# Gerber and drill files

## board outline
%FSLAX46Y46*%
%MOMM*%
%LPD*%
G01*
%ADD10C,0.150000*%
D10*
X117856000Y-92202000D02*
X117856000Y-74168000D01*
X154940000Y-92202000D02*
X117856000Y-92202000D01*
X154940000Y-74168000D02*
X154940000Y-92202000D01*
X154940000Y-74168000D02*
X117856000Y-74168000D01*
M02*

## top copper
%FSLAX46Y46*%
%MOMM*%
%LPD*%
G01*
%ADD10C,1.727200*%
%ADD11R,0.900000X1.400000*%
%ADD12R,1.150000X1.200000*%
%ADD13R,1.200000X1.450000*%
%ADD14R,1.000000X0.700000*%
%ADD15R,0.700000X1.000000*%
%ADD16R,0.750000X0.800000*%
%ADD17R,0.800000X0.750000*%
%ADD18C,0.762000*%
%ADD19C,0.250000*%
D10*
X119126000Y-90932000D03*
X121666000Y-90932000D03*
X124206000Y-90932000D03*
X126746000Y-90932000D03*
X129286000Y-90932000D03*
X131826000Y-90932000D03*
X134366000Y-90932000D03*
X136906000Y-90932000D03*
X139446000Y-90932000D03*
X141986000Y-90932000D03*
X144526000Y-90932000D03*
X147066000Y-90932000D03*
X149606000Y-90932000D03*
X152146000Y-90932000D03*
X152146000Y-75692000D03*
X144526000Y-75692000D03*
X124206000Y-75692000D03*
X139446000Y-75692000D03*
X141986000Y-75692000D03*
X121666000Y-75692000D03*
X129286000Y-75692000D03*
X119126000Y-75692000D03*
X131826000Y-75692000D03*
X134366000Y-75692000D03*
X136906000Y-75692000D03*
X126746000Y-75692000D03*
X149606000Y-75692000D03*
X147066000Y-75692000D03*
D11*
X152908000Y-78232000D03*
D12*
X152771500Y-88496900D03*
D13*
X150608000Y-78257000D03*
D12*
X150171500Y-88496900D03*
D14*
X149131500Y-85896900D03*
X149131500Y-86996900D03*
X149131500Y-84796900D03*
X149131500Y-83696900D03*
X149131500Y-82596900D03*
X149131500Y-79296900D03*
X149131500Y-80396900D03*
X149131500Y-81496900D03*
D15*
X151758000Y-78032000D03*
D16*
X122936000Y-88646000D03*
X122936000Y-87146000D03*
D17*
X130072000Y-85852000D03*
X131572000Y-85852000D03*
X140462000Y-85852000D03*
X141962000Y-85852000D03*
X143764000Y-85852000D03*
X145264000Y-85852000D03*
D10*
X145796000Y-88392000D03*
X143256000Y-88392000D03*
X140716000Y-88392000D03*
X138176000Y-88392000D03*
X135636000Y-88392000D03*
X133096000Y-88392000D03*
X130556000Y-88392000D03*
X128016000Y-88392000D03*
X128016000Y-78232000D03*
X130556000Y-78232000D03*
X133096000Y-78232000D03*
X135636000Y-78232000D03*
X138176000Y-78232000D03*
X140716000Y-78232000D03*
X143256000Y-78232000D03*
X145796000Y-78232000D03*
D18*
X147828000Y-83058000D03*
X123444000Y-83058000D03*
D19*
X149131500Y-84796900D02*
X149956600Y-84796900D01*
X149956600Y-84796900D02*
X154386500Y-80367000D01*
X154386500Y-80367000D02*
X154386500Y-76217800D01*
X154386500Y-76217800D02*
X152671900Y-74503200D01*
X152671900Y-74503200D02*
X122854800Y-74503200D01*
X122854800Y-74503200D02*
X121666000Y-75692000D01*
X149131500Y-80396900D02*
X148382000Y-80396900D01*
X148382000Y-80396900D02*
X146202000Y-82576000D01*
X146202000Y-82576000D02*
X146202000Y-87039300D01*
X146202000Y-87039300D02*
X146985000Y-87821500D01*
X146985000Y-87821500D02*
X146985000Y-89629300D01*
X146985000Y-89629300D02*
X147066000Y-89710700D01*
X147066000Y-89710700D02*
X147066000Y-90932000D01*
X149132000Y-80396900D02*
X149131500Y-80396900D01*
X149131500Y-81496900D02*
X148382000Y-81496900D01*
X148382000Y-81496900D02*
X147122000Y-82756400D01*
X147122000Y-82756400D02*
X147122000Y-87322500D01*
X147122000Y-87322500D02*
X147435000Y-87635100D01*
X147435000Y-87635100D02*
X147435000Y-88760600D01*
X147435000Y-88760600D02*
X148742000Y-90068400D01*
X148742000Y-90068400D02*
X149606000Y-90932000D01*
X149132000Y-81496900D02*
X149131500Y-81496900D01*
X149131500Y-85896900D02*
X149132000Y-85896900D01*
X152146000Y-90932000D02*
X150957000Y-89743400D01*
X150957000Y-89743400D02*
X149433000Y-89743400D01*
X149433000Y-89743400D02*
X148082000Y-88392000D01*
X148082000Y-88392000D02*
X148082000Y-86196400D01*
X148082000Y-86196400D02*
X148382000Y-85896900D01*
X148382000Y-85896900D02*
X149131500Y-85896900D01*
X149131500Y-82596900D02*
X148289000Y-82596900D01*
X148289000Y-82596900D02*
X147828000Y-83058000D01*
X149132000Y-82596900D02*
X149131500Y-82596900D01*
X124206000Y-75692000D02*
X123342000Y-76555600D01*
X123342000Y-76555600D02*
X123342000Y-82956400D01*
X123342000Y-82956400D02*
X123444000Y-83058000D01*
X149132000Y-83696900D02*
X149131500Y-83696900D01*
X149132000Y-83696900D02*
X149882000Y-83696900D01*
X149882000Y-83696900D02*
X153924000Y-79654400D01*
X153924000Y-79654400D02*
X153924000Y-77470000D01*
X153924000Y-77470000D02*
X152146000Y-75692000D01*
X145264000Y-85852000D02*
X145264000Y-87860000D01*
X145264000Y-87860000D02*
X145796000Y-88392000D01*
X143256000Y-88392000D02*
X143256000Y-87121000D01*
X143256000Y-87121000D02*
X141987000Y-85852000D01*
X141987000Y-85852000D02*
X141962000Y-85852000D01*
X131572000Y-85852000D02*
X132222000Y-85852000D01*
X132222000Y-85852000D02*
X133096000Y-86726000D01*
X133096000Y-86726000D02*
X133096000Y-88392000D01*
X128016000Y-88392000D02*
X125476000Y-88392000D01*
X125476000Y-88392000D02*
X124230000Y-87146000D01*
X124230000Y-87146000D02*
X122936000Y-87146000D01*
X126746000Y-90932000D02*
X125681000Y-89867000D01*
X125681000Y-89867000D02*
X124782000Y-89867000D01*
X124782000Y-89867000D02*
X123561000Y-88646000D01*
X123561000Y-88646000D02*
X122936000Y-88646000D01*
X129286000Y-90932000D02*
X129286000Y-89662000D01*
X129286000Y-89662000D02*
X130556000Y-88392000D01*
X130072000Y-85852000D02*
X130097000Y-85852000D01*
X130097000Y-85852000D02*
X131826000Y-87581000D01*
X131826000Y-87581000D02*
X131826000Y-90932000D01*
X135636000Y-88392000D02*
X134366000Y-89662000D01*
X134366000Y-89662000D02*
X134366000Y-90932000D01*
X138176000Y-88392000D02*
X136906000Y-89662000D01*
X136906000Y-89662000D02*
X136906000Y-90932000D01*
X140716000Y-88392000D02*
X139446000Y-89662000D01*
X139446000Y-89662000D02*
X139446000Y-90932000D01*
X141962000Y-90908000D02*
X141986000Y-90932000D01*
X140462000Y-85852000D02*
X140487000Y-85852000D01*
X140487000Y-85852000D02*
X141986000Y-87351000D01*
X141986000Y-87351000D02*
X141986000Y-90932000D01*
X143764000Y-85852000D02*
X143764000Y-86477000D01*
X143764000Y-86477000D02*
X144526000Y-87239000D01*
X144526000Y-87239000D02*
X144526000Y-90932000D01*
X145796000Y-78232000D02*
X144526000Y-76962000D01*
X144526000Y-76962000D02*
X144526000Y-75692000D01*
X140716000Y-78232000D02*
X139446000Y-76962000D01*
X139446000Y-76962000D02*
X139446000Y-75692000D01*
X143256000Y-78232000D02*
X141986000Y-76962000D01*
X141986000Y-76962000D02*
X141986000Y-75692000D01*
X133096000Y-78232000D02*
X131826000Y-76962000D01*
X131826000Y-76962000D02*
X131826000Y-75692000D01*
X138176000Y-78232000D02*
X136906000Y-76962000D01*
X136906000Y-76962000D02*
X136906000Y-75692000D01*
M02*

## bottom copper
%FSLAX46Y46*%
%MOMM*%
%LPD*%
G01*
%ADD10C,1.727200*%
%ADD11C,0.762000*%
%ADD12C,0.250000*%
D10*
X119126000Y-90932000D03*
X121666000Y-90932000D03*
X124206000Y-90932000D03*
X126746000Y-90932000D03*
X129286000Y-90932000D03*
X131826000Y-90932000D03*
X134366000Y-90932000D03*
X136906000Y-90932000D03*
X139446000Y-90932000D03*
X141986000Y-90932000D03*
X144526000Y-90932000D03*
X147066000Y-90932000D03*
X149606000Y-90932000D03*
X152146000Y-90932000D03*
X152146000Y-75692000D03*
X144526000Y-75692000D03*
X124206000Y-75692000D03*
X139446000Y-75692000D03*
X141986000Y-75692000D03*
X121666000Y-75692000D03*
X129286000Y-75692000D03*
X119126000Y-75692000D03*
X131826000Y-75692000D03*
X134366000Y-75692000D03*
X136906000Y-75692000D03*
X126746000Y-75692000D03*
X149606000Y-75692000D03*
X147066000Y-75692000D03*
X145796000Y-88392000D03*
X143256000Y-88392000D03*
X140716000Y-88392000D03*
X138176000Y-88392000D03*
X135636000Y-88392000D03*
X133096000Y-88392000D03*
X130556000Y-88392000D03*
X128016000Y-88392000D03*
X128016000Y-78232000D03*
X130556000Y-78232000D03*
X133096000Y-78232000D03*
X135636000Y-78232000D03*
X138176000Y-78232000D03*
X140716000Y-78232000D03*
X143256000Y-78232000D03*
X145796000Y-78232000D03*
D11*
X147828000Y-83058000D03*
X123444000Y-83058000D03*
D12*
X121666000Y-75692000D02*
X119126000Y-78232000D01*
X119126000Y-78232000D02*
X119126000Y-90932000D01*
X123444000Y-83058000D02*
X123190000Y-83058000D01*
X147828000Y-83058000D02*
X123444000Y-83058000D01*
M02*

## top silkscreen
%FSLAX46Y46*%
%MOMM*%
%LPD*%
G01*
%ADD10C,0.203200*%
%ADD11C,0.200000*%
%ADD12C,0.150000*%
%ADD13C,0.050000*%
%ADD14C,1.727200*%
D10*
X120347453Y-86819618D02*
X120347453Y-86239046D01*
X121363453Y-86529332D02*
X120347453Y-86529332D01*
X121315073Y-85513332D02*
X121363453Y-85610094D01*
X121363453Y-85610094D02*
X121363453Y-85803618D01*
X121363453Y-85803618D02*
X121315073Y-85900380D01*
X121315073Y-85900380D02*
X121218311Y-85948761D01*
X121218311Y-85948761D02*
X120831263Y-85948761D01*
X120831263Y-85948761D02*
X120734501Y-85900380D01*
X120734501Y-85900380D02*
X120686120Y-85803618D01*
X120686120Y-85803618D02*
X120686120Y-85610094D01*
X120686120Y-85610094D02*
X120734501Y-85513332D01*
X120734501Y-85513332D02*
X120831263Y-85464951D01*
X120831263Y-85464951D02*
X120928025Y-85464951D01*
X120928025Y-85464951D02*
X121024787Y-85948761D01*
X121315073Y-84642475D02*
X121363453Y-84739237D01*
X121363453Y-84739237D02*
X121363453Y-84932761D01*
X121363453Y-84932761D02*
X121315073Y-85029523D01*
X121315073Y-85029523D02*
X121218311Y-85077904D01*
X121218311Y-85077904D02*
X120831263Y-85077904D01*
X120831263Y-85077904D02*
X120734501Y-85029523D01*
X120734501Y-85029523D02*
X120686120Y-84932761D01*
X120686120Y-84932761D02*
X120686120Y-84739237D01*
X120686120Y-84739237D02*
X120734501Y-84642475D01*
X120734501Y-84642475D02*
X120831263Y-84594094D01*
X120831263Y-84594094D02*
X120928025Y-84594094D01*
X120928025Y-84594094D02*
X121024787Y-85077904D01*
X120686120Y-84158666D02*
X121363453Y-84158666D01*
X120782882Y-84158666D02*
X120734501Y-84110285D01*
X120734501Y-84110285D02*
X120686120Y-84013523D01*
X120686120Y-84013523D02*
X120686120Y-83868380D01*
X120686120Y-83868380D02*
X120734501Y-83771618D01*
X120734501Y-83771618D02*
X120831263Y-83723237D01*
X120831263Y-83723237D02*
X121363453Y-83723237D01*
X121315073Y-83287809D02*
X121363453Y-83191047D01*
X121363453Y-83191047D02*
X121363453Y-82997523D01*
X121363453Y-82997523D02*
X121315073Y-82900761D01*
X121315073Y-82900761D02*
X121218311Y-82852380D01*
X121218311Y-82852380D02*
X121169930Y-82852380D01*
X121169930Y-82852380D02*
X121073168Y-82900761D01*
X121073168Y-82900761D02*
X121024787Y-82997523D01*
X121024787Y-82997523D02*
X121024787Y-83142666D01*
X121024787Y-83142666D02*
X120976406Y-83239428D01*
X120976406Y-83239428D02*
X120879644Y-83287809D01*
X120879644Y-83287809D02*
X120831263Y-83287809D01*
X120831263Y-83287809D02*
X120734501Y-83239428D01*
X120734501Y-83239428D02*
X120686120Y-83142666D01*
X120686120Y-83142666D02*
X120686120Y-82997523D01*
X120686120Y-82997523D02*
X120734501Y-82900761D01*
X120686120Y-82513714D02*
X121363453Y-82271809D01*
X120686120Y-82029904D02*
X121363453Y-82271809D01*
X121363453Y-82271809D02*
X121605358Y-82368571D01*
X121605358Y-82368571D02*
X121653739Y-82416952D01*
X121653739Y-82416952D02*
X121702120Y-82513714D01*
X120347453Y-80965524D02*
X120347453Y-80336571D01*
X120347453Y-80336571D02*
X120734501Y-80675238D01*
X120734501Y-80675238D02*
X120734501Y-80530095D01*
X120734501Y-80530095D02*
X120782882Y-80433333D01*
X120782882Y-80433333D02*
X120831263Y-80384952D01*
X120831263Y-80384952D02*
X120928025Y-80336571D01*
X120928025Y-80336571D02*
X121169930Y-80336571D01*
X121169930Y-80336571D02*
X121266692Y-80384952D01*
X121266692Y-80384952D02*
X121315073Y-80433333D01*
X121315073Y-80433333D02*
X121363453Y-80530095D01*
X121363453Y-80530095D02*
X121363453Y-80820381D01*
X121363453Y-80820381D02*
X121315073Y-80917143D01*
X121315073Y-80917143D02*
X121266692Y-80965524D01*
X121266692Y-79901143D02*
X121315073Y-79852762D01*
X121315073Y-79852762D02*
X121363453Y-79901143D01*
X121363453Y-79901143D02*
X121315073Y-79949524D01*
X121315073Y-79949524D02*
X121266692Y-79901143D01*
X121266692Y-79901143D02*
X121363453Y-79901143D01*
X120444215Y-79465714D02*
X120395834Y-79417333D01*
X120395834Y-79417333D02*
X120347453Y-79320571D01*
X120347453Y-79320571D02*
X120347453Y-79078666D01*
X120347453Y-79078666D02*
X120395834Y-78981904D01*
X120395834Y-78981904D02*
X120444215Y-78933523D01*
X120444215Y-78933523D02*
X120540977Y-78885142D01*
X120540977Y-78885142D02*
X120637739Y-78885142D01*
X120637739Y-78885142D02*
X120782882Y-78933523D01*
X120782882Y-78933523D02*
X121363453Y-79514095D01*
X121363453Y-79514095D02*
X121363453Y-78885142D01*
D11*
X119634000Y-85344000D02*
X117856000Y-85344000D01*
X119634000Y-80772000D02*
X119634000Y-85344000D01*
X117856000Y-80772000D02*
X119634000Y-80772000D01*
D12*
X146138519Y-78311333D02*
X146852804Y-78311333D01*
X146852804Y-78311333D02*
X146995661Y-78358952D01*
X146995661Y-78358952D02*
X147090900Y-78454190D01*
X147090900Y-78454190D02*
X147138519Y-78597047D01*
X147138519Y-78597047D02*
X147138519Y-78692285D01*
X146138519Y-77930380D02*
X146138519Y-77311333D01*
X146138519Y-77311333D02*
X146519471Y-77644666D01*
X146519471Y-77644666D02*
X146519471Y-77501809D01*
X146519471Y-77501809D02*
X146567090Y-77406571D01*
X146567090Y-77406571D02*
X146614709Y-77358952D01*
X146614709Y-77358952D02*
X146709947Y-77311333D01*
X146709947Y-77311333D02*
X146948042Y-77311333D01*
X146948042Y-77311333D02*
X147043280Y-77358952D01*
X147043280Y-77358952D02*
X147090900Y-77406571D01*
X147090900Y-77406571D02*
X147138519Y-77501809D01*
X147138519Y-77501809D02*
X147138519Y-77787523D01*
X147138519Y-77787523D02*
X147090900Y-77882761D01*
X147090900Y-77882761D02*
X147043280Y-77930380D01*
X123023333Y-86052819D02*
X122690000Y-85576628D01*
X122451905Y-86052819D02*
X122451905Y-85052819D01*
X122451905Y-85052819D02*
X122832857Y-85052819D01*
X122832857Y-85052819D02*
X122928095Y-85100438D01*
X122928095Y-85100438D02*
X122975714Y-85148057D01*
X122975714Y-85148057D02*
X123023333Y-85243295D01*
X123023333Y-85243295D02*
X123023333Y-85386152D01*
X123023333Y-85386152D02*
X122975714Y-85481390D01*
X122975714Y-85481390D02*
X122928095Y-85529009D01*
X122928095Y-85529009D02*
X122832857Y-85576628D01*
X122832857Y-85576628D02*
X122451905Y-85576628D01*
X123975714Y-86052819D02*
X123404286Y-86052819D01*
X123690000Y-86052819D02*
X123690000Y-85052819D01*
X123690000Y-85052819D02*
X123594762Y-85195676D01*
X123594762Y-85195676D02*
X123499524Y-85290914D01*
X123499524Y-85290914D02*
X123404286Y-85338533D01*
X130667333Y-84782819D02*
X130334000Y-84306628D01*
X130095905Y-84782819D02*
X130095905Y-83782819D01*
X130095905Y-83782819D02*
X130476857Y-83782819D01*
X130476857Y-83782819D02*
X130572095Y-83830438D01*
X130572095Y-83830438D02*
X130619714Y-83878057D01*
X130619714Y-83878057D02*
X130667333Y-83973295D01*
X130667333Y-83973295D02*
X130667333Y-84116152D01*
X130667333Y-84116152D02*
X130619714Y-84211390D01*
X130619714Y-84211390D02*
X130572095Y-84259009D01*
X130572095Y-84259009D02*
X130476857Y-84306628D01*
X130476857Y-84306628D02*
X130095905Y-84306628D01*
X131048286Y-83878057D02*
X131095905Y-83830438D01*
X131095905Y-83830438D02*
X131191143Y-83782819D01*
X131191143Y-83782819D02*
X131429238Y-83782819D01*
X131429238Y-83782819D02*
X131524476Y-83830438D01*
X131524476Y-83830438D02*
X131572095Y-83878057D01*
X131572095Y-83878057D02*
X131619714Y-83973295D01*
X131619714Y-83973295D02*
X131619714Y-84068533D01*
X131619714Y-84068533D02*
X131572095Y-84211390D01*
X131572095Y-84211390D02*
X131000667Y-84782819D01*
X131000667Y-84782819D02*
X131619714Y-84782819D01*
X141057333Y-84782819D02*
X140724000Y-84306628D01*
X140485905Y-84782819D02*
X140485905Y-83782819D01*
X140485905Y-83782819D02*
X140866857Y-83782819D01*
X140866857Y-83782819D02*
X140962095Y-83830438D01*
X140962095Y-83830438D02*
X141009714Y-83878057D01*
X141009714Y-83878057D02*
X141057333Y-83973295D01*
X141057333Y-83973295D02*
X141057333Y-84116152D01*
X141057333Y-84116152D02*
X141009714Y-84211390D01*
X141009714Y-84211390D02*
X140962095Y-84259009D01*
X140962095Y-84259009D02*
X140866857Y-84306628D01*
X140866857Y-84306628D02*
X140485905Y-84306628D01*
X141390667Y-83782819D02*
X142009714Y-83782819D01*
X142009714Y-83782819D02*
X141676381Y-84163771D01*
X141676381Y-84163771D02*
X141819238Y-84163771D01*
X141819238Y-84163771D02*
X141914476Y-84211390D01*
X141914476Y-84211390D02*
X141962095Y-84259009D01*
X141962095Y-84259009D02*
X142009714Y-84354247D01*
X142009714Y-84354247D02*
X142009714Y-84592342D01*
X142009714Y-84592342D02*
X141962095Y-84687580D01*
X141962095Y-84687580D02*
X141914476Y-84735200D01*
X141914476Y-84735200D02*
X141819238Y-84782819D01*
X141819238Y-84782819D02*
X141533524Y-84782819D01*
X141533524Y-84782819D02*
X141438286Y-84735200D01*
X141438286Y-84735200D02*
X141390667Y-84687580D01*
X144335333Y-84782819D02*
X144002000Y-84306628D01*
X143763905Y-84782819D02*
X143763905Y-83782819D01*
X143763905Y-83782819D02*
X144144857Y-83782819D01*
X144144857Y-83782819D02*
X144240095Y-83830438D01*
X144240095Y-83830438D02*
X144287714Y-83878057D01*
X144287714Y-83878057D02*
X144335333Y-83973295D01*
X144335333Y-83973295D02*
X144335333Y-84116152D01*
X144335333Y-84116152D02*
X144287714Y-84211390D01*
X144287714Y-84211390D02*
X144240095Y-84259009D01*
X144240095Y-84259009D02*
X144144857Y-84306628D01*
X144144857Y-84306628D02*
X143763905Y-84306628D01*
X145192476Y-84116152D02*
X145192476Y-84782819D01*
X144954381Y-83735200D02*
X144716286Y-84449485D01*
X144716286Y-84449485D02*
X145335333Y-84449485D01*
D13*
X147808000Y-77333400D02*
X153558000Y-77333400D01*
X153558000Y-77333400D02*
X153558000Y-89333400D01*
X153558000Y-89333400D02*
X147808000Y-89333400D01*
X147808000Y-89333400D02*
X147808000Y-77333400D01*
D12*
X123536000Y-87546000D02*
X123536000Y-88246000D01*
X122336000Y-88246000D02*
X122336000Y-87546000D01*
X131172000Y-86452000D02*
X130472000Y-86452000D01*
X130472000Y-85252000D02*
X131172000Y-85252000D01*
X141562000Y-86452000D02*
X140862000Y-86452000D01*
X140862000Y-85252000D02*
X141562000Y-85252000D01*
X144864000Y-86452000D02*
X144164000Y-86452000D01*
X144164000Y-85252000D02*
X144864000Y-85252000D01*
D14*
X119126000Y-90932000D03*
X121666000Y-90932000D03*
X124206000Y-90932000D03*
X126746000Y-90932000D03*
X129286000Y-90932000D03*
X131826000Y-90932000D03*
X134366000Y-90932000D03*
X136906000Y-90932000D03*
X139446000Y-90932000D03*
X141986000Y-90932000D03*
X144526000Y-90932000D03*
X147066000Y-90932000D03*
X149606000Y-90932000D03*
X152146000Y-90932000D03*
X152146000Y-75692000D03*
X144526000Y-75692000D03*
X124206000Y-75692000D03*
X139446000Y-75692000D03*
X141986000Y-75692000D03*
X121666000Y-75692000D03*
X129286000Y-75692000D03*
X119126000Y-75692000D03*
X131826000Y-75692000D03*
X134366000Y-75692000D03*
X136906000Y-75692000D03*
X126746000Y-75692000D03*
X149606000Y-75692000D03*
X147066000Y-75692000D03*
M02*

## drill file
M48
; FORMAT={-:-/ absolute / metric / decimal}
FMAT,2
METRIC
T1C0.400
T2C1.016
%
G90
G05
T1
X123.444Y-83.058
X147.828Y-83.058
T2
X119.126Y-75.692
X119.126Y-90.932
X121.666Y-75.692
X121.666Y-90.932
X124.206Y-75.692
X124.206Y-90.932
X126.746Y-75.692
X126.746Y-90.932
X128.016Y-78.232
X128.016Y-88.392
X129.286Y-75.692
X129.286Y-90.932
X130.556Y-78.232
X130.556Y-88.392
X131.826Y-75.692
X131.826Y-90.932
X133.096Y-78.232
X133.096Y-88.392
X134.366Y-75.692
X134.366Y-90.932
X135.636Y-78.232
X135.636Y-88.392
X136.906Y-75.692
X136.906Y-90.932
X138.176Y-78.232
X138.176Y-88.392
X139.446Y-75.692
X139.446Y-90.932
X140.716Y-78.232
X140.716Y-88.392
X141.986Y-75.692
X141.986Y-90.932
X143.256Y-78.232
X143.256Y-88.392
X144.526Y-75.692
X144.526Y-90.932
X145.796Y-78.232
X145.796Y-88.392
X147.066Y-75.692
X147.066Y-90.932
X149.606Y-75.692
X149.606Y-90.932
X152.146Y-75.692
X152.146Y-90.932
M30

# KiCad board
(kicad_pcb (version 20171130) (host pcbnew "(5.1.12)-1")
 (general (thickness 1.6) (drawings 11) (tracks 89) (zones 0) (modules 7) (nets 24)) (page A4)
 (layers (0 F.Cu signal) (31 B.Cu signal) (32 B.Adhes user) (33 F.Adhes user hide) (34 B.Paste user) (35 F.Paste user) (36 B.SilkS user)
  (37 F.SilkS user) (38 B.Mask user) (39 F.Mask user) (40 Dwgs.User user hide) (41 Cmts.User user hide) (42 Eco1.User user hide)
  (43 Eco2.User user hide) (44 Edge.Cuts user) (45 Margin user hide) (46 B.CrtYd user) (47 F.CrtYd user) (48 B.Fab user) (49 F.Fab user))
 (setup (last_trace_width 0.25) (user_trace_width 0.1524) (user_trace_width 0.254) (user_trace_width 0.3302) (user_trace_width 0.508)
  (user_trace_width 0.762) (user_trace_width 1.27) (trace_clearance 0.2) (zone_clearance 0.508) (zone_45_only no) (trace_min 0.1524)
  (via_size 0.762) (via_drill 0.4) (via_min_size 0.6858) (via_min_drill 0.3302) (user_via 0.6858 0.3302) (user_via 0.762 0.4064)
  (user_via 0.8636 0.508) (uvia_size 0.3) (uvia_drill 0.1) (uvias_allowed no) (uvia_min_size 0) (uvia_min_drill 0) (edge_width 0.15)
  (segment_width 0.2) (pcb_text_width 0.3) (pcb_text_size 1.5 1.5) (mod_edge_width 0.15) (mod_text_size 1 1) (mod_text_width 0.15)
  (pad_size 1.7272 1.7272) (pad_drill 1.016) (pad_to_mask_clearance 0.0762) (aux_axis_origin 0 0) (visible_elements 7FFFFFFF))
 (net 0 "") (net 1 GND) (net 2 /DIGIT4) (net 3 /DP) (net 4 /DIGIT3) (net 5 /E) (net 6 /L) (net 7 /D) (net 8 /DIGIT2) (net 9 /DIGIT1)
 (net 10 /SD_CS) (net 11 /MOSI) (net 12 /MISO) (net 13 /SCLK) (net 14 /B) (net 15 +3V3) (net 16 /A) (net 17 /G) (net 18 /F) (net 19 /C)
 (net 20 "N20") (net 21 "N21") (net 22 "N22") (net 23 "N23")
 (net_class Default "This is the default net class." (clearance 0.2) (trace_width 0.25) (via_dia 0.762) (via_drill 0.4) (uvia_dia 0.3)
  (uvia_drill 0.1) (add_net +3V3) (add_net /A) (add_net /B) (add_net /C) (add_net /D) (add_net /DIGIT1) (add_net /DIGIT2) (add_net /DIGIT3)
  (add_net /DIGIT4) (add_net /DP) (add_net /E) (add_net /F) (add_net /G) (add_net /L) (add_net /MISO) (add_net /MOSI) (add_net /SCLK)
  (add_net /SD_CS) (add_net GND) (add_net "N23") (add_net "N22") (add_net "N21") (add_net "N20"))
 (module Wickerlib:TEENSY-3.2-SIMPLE (layer F.Cu) (at 129.286 80.772 90)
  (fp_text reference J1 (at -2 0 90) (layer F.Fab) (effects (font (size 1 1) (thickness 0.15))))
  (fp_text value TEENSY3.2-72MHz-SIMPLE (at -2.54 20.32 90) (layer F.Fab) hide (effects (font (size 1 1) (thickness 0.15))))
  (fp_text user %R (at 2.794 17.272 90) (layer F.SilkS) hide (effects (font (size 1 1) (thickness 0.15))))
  (pad G1 thru_hole circle (at -10.16 -10.16 90) (size 1.7272 1.7272) (drill 1.016) (layers *.Cu *.Mask F.SilkS) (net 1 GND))
  (pad 0 thru_hole circle (at -10.16 -7.62 90) (size 1.7272 1.7272) (drill 1.016) (layers *.Cu *.Mask F.SilkS))
  (pad 1 thru_hole circle (at -10.16 -5.08 90) (size 1.7272 1.7272) (drill 1.016) (layers *.Cu *.Mask F.SilkS))
  (pad 2 thru_hole circle (at -10.16 -2.54 90) (size 1.7272 1.7272) (drill 1.016) (layers *.Cu *.Mask F.SilkS) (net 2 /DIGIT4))
  (pad 3 thru_hole circle (at -10.16 0 90) (size 1.7272 1.7272) (drill 1.016) (layers *.Cu *.Mask F.SilkS) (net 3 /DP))
  (pad 4 thru_hole circle (at -10.16 2.54 90) (size 1.7272 1.7272) (drill 1.016) (layers *.Cu *.Mask F.SilkS) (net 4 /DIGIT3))
  (pad 5 thru_hole circle (at -10.16 5.08 90) (size 1.7272 1.7272) (drill 1.016) (layers *.Cu *.Mask F.SilkS) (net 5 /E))
  (pad 6 thru_hole circle (at -10.16 7.62 90) (size 1.7272 1.7272) (drill 1.016) (layers *.Cu *.Mask F.SilkS) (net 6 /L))
  (pad 7 thru_hole circle (at -10.16 10.16 90) (size 1.7272 1.7272) (drill 1.016) (layers *.Cu *.Mask F.SilkS) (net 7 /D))
  (pad 8 thru_hole circle (at -10.16 12.7 90) (size 1.7272 1.7272) (drill 1.016) (layers *.Cu *.Mask F.SilkS) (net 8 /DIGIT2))
  (pad 9 thru_hole circle (at -10.16 15.24 90) (size 1.7272 1.7272) (drill 1.016) (layers *.Cu *.Mask F.SilkS) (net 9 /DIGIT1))
  (pad 10 thru_hole circle (at -10.16 17.78 90) (size 1.7272 1.7272) (drill 1.016) (layers *.Cu *.Mask F.SilkS) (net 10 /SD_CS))
  (pad 11 thru_hole circle (at -10.16 20.32 90) (size 1.7272 1.7272) (drill 1.016) (layers *.Cu *.Mask F.SilkS) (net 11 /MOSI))
  (pad 12 thru_hole circle (at -10.16 22.86 90) (size 1.7272 1.7272) (drill 1.016) (layers *.Cu *.Mask F.SilkS) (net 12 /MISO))
  (pad 13 thru_hole circle (at 5.08 22.86 90) (size 1.7272 1.7272) (drill 1.016) (layers *.Cu *.Mask F.SilkS) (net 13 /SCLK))
  (pad 16 thru_hole circle (at 5.08 15.24 90) (size 1.7272 1.7272) (drill 1.016) (layers *.Cu *.Mask F.SilkS) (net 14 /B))
  (pad 3V2 thru_hole circle (at 5.08 -5.08 90) (size 1.7272 1.7272) (drill 1.016) (layers *.Cu *.Mask F.SilkS) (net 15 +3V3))
  (pad 18 thru_hole circle (at 5.08 10.16 90) (size 1.7272 1.7272) (drill 1.016) (layers *.Cu *.Mask F.SilkS) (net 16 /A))
  (pad 17 thru_hole circle (at 5.08 12.7 90) (size 1.7272 1.7272) (drill 1.016) (layers *.Cu *.Mask F.SilkS) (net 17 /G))
  (pad AG thru_hole circle (at 5.08 -7.62 90) (size 1.7272 1.7272) (drill 1.016) (layers *.Cu *.Mask F.SilkS) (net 1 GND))
  (pad 22 thru_hole circle (at 5.08 0 90) (size 1.7272 1.7272) (drill 1.016) (layers *.Cu *.Mask F.SilkS))
  (pad VIN thru_hole circle (at 5.08 -10.16 90) (size 1.7272 1.7272) (drill 1.016) (layers *.Cu *.Mask F.SilkS))
  (pad 21 thru_hole circle (at 5.08 2.54 90) (size 1.7272 1.7272) (drill 1.016) (layers *.Cu *.Mask F.SilkS) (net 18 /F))
  (pad 20 thru_hole circle (at 5.08 5.08 90) (size 1.7272 1.7272) (drill 1.016) (layers *.Cu *.Mask F.SilkS))
  (pad 19 thru_hole circle (at 5.08 7.62 90) (size 1.7272 1.7272) (drill 1.016) (layers *.Cu *.Mask F.SilkS) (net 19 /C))
  (pad 23 thru_hole circle (at 5.08 -2.54 90) (size 1.7272 1.7272) (drill 1.016) (layers *.Cu *.Mask F.SilkS))
  (pad 14 thru_hole circle (at 5.08 20.32 90) (size 1.7272 1.7272) (drill 1.016) (layers *.Cu *.Mask F.SilkS))
  (pad 15 thru_hole circle (at 5.08 17.78 90) (size 1.7272 1.7272) (drill 1.016) (layers *.Cu *.Mask F.SilkS)))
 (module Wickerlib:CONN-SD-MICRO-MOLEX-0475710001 (layer F.Cu) (at 147.808 83.0834 90)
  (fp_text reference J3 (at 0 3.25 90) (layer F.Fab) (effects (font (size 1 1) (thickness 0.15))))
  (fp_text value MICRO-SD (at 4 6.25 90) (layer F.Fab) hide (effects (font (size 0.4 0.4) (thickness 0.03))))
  (fp_line (start 5.75 0) (end 5.75 5.75) (layer F.SilkS) (width 0.05))
  (fp_line (start 5.75 5.75) (end -6.25 5.75) (layer F.SilkS) (width 0.05))
  (fp_line (start -6.25 5.75) (end -6.25 0) (layer F.SilkS) (width 0.05))
  (fp_line (start -6.25 0) (end 5.75 0) (layer F.SilkS) (width 0.05))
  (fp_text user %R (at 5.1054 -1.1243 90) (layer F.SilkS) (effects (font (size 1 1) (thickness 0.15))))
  (pad G5 smd rect (at 4.8514 5.1 90) (size 1.4 0.9) (layers F.Cu F.Paste F.Mask))
  (pad G2 smd rect (at -5.4135 4.9635 90) (size 1.2 1.15) (layers F.Cu F.Paste F.Mask))
  (pad G3 smd rect (at 4.8264 2.8 90) (size 1.45 1.2) (layers F.Cu F.Paste F.Mask))
  (pad G1 smd rect (at -5.4135 2.3635 90) (size 1.2 1.15) (layers F.Cu F.Paste F.Mask))
  (pad 7 smd rect (at -2.8135 1.3235 90) (size 0.7 1) (layers F.Cu F.Paste F.Mask) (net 12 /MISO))
  (pad 8 smd rect (at -3.9135 1.3235 90) (size 0.7 1) (layers F.Cu F.Paste F.Mask))
  (pad 6 smd rect (at -1.7135 1.3235 90) (size 0.7 1) (layers F.Cu F.Paste F.Mask) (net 1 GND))
  (pad 5 smd rect (at -0.6135 1.3235 90) (size 0.7 1) (layers F.Cu F.Paste F.Mask) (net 13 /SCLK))
  (pad 4 smd rect (at 0.4865 1.3235 90) (size 0.7 1) (layers F.Cu F.Paste F.Mask) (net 15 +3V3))
  (pad 1 smd rect (at 3.7865 1.3235 90) (size 0.7 1) (layers F.Cu F.Paste F.Mask))
  (pad 2 smd rect (at 2.6865 1.3235 90) (size 0.7 1) (layers F.Cu F.Paste F.Mask) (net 10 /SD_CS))
  (pad 3 smd rect (at 1.5865 1.3235 90) (size 0.7 1) (layers F.Cu F.Paste F.Mask) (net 11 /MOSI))
  (pad G4 smd rect (at 5.0514 3.95 90) (size 1 0.7) (layers F.Cu F.Paste F.Mask)))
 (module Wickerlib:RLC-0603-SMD (layer F.Cu) (at 122.936 87.896 90)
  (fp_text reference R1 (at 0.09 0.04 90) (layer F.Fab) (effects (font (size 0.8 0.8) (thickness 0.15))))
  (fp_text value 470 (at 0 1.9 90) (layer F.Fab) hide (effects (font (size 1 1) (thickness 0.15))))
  (fp_line (start 0.35 0.6) (end -0.35 0.6) (layer F.SilkS) (width 0.15))
  (fp_line (start -0.35 -0.6) (end 0.35 -0.6) (layer F.SilkS) (width 0.15))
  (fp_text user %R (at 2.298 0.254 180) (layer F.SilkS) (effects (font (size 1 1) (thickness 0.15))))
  (pad 1 smd rect (at -0.75 0 90) (size 0.8 0.75) (layers F.Cu F.Paste F.Mask) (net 2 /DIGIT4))
  (pad 2 smd rect (at 0.75 0 90) (size 0.8 0.75) (layers F.Cu F.Paste F.Mask) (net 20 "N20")))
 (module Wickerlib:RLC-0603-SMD (layer F.Cu) (at 130.822 85.852)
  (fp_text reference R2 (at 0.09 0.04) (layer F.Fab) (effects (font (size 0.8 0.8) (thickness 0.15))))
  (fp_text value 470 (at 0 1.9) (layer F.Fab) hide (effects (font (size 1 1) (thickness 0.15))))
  (fp_line (start 0.35 0.6) (end -0.35 0.6) (layer F.SilkS) (width 0.15))
  (fp_line (start -0.35 -0.6) (end 0.35 -0.6) (layer F.SilkS) (width 0.15))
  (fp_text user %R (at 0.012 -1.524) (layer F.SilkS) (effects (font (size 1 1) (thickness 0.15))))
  (pad 1 smd rect (at -0.75 0) (size 0.8 0.75) (layers F.Cu F.Paste F.Mask) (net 4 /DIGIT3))
  (pad 2 smd rect (at 0.75 0) (size 0.8 0.75) (layers F.Cu F.Paste F.Mask) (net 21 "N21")))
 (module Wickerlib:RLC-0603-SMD (layer F.Cu) (at 141.212 85.852)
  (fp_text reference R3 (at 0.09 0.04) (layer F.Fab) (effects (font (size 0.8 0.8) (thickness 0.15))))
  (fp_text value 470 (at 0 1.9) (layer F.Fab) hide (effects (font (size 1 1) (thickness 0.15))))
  (fp_line (start 0.35 0.6) (end -0.35 0.6) (layer F.SilkS) (width 0.15))
  (fp_line (start -0.35 -0.6) (end 0.35 -0.6) (layer F.SilkS) (width 0.15))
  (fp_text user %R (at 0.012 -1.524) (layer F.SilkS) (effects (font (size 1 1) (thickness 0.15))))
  (pad 1 smd rect (at -0.75 0) (size 0.8 0.75) (layers F.Cu F.Paste F.Mask) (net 8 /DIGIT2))
  (pad 2 smd rect (at 0.75 0) (size 0.8 0.75) (layers F.Cu F.Paste F.Mask) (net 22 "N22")))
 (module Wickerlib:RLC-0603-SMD (layer F.Cu) (at 144.514 85.852)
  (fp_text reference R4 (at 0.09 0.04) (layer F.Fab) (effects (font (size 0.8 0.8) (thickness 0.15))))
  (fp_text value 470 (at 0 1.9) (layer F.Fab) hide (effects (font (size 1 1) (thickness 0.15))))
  (fp_line (start 0.35 0.6) (end -0.35 0.6) (layer F.SilkS) (width 0.15))
  (fp_line (start -0.35 -0.6) (end 0.35 -0.6) (layer F.SilkS) (width 0.15))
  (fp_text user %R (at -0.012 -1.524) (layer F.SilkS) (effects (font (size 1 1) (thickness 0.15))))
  (pad 1 smd rect (at -0.75 0) (size 0.8 0.75) (layers F.Cu F.Paste F.Mask) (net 9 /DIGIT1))
  (pad 2 smd rect (at 0.75 0) (size 0.8 0.75) (layers F.Cu F.Paste F.Mask) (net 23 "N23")))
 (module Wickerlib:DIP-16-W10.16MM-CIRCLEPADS (layer B.Cu) (at 137.046 84.142 90)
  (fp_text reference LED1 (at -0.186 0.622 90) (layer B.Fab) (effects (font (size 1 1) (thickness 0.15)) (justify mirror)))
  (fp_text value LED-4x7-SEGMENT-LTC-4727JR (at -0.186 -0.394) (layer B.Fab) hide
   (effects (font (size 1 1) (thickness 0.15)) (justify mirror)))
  (pad 1 thru_hole circle (at -4.25 8.75 90) (size 1.7272 1.7272) (drill 1.016) (layers *.Cu *.Mask B.SilkS) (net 23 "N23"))
  (pad 2 thru_hole circle (at -4.25 6.21 90) (size 1.7272 1.7272) (drill 1.016) (layers *.Cu *.Mask B.SilkS) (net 22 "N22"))
  (pad 3 thru_hole circle (at -4.25 3.67 90) (size 1.7272 1.7272) (drill 1.016) (layers *.Cu *.Mask B.SilkS) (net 7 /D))
  (pad 4 thru_hole circle (at -4.25 1.13 90) (size 1.7272 1.7272) (drill 1.016) (layers *.Cu *.Mask B.SilkS) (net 6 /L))
  (pad 5 thru_hole circle (at -4.25 -1.41 90) (size 1.7272 1.7272) (drill 1.016) (layers *.Cu *.Mask B.SilkS) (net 5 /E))
  (pad 6 thru_hole circle (at -4.25 -3.95 90) (size 1.7272 1.7272) (drill 1.016) (layers *.Cu *.Mask B.SilkS) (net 21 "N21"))
  (pad 7 thru_hole circle (at -4.25 -6.49 90) (size 1.7272 1.7272) (drill 1.016) (layers *.Cu *.Mask B.SilkS) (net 3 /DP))
  (pad 8 thru_hole circle (at -4.25 -9.03 90) (size 1.7272 1.7272) (drill 1.016) (layers *.Cu *.Mask B.SilkS) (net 20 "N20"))
  (pad 9 thru_hole circle (at 5.91 -9.03 90) (size 1.7272 1.7272) (drill 1.016) (layers *.Cu *.Mask B.SilkS))
  (pad 10 thru_hole circle (at 5.91 -6.49 90) (size 1.7272 1.7272) (drill 1.016) (layers *.Cu *.Mask B.SilkS))
  (pad 11 thru_hole circle (at 5.91 -3.95 90) (size 1.7272 1.7272) (drill 1.016) (layers *.Cu *.Mask B.SilkS) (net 18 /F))
  (pad 12 thru_hole circle (at 5.91 -1.41 90) (size 1.7272 1.7272) (drill 1.016) (layers *.Cu *.Mask B.SilkS))
  (pad 13 thru_hole circle (at 5.91 1.13 90) (size 1.7272 1.7272) (drill 1.016) (layers *.Cu *.Mask B.SilkS) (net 19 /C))
  (pad 14 thru_hole circle (at 5.91 3.67 90) (size 1.7272 1.7272) (drill 1.016) (layers *.Cu *.Mask B.SilkS) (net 16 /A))
  (pad 15 thru_hole circle (at 5.91 6.21 90) (size 1.7272 1.7272) (drill 1.016) (layers *.Cu *.Mask B.SilkS) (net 17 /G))
  (pad 16 thru_hole circle (at 5.91 8.75 90) (size 1.7272 1.7272) (drill 1.016) (layers *.Cu *.Mask B.SilkS) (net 14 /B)))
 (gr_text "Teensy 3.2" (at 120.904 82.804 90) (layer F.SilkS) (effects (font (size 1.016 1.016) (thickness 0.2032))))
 (gr_line (start 119.634 85.344) (end 117.856 85.344) (layer F.SilkS) (width 0.2))
 (gr_line (start 119.634 80.772) (end 119.634 85.344) (layer F.SilkS) (width 0.2))
 (gr_line (start 117.856 80.772) (end 119.634 80.772) (layer F.SilkS) (width 0.2))
 (gr_line (start 117.856 92.202) (end 117.856 74.168) (layer Edge.Cuts) (width 0.15))
 (gr_line (start 154.94 92.202) (end 117.856 92.202) (layer Edge.Cuts) (width 0.15))
 (gr_line (start 154.94 74.168) (end 154.94 92.202) (layer Edge.Cuts) (width 0.15))
 (gr_line (start 154.94 74.168) (end 117.856 74.168) (layer Edge.Cuts) (width 0.15))
 (segment (start 121.666 75.692) (end 119.126 78.232) (width 0.25) (layer B.Cu) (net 1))
 (segment (start 119.126 78.232) (end 119.126 90.932) (width 0.25) (layer B.Cu) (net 1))
 (segment (start 149.1315 84.7969) (end 149.9566 84.7969) (width 0.25) (layer F.Cu) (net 1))
 (segment (start 149.9566 84.7969) (end 154.3865 80.367) (width 0.25) (layer F.Cu) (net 1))
 (segment (start 154.3865 80.367) (end 154.3865 76.2178) (width 0.25) (layer F.Cu) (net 1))
 (segment (start 154.3865 76.2178) (end 152.6719 74.5032) (width 0.25) (layer F.Cu) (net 1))
 (segment (start 152.6719 74.5032) (end 122.8548 74.5032) (width 0.25) (layer F.Cu) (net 1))
 (segment (start 122.8548 74.5032) (end 121.666 75.692) (width 0.25) (layer F.Cu) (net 1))
 (segment (start 149.1315 80.3969) (end 148.382 80.3969) (width 0.25) (layer F.Cu) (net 10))
 (segment (start 148.382 80.3969) (end 146.202 82.576) (width 0.25) (layer F.Cu) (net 10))
 (segment (start 146.202 82.576) (end 146.202 87.0393) (width 0.25) (layer F.Cu) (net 10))
 (segment (start 146.202 87.0393) (end 146.985 87.8215) (width 0.25) (layer F.Cu) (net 10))
 (segment (start 146.985 87.8215) (end 146.985 89.6293) (width 0.25) (layer F.Cu) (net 10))
 (segment (start 146.985 89.6293) (end 147.066 89.7107) (width 0.25) (layer F.Cu) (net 10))
 (segment (start 147.066 89.7107) (end 147.066 90.932) (width 0.25) (layer F.Cu) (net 10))
 (segment (start 149.132 80.3969) (end 149.1315 80.3969) (width 0.25) (layer F.Cu) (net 10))
 (segment (start 149.1315 81.4969) (end 148.382 81.4969) (width 0.25) (layer F.Cu) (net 11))
 (segment (start 148.382 81.4969) (end 147.122 82.7564) (width 0.25) (layer F.Cu) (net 11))
 (segment (start 147.122 82.7564) (end 147.122 87.3225) (width 0.25) (layer F.Cu) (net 11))
 (segment (start 147.122 87.3225) (end 147.435 87.6351) (width 0.25) (layer F.Cu) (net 11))
 (segment (start 147.435 87.6351) (end 147.435 88.7606) (width 0.25) (layer F.Cu) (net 11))
 (segment (start 147.435 88.7606) (end 148.742 90.0684) (width 0.25) (layer F.Cu) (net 11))
 (segment (start 148.742 90.0684) (end 149.606 90.932) (width 0.25) (layer F.Cu) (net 11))
 (segment (start 149.132 81.4969) (end 149.1315 81.4969) (width 0.25) (layer F.Cu) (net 11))
 (segment (start 149.1315 85.8969) (end 149.132 85.8969) (width 0.25) (layer F.Cu) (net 12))
 (segment (start 152.146 90.932) (end 150.957 89.7434) (width 0.25) (layer F.Cu) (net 12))
 (segment (start 150.957 89.7434) (end 149.433 89.7434) (width 0.25) (layer F.Cu) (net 12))
 (segment (start 149.433 89.7434) (end 148.082 88.392) (width 0.25) (layer F.Cu) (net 12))
 (segment (start 148.082 88.392) (end 148.082 86.1964) (width 0.25) (layer F.Cu) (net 12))
 (segment (start 148.082 86.1964) (end 148.382 85.8969) (width 0.25) (layer F.Cu) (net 12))
 (segment (start 148.382 85.8969) (end 149.1315 85.8969) (width 0.25) (layer F.Cu) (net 12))
 (segment (start 123.444 83.058) (end 123.19 83.058) (width 0.25) (layer B.Cu) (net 15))
 (segment (start 147.828 83.058) (end 123.444 83.058) (width 0.25) (layer B.Cu) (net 15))
 (segment (start 149.1315 82.5969) (end 148.289 82.5969) (width 0.25) (layer F.Cu) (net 15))
 (segment (start 148.289 82.5969) (end 147.828 83.058) (width 0.25) (layer F.Cu) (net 15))
 (segment (start 149.132 82.5969) (end 149.1315 82.5969) (width 0.25) (layer F.Cu) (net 15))
 (segment (start 124.206 75.692) (end 123.342 76.5556) (width 0.25) (layer F.Cu) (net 15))
 (segment (start 123.342 76.5556) (end 123.342 82.9564) (width 0.25) (layer F.Cu) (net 15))
 (segment (start 123.342 82.9564) (end 123.444 83.058) (width 0.25) (layer F.Cu) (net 15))
 (via (at 147.828 83.058) (size 0.762) (layers F.Cu B.Cu) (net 15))
 (via (at 123.444 83.058) (size 0.762) (layers F.Cu B.Cu) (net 15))
 (segment (start 149.132 83.6969) (end 149.1315 83.6969) (width 0.25) (layer F.Cu) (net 13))
 (segment (start 149.132 83.6969) (end 149.882 83.6969) (width 0.25) (layer F.Cu) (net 13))
 (segment (start 149.882 83.6969) (end 153.924 79.6544) (width 0.25) (layer F.Cu) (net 13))
 (segment (start 153.924 79.6544) (end 153.924 77.47) (width 0.25) (layer F.Cu) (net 13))
 (segment (start 153.924 77.47) (end 152.146 75.692) (width 0.25) (layer F.Cu) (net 13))
 (segment (start 145.264 85.852) (end 145.264 87.86) (width 0.25) (layer F.Cu) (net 23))
 (segment (start 145.264 87.86) (end 145.796 88.392) (width 0.25) (layer F.Cu) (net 23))
 (segment (start 143.256 88.392) (end 143.256 87.121) (width 0.25) (layer F.Cu) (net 22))
 (segment (start 143.256 87.121) (end 141.987 85.852) (width 0.25) (layer F.Cu) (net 22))
 (segment (start 141.987 85.852) (end 141.962 85.852) (width 0.25) (layer F.Cu) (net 22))
 (segment (start 131.572 85.852) (end 132.222 85.852) (width 0.25) (layer F.Cu) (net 21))
 (segment (start 132.222 85.852) (end 133.096 86.726) (width 0.25) (layer F.Cu) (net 21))
 (segment (start 133.096 86.726) (end 133.096 88.392) (width 0.25) (layer F.Cu) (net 21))
 (segment (start 128.016 88.392) (end 125.476 88.392) (width 0.25) (layer F.Cu) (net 20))
 (segment (start 125.476 88.392) (end 124.23 87.146) (width 0.25) (layer F.Cu) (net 20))
 (segment (start 124.23 87.146) (end 122.936 87.146) (width 0.25) (layer F.Cu) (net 20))
 (segment (start 126.746 90.932) (end 125.681 89.867) (width 0.25) (layer F.Cu) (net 2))
 (segment (start 125.681 89.867) (end 124.782 89.867) (width 0.25) (layer F.Cu) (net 2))
 (segment (start 124.782 89.867) (end 123.561 88.646) (width 0.25) (layer F.Cu) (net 2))
 (segment (start 123.561 88.646) (end 122.936 88.646) (width 0.25) (layer F.Cu) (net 2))
 (segment (start 129.286 90.932) (end 129.286 89.662) (width 0.25) (layer F.Cu) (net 3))
 (segment (start 129.286 89.662) (end 130.556 88.392) (width 0.25) (layer F.Cu) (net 3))
 (segment (start 130.072 85.852) (end 130.097 85.852) (width 0.25) (layer F.Cu) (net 4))
 (segment (start 130.097 85.852) (end 131.826 87.581) (width 0.25) (layer F.Cu) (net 4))
 (segment (start 131.826 87.581) (end 131.826 90.932) (width 0.25) (layer F.Cu) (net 4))
 (segment (start 135.636 88.392) (end 134.366 89.662) (width 0.25) (layer F.Cu) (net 5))
 (segment (start 134.366 89.662) (end 134.366 90.932) (width 0.25) (layer F.Cu) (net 5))
 (segment (start 138.176 88.392) (end 136.906 89.662) (width 0.25) (layer F.Cu) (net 6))
 (segment (start 136.906 89.662) (end 136.906 90.932) (width 0.25) (layer F.Cu) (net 6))
 (segment (start 140.716 88.392) (end 139.446 89.662) (width 0.25) (layer F.Cu) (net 7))
 (segment (start 139.446 89.662) (end 139.446 90.932) (width 0.25) (layer F.Cu) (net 7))
 (segment (start 141.962 90.908) (end 141.986 90.932) (width 0.25) (layer F.Cu) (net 8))
 (segment (start 140.462 85.852) (end 140.487 85.852) (width 0.25) (layer F.Cu) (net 8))
 (segment (start 140.487 85.852) (end 141.986 87.351) (width 0.25) (layer F.Cu) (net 8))
 (segment (start 141.986 87.351) (end 141.986 90.932) (width 0.25) (layer F.Cu) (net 8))
 (segment (start 143.764 85.852) (end 143.764 86.477) (width 0.25) (layer F.Cu) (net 9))
 (segment (start 143.764 86.477) (end 144.526 87.239) (width 0.25) (layer F.Cu) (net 9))
 (segment (start 144.526 87.239) (end 144.526 90.932) (width 0.25) (layer F.Cu) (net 9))
 (segment (start 145.796 78.232) (end 144.526 76.962) (width 0.25) (layer F.Cu) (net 14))
 (segment (start 144.526 76.962) (end 144.526 75.692) (width 0.25) (layer F.Cu) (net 14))
 (segment (start 140.716 78.232) (end 139.446 76.962) (width 0.25) (layer F.Cu) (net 16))
 (segment (start 139.446 76.962) (end 139.446 75.692) (width 0.25) (layer F.Cu) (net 16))
 (segment (start 143.256 78.232) (end 141.986 76.962) (width 0.25) (layer F.Cu) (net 17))
 (segment (start 141.986 76.962) (end 141.986 75.692) (width 0.25) (layer F.Cu) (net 17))
 (segment (start 133.096 78.232) (end 131.826 76.962) (width 0.25) (layer F.Cu) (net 18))
 (segment (start 131.826 76.962) (end 131.826 75.692) (width 0.25) (layer F.Cu) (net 18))
 (segment (start 138.176 78.232) (end 136.906 76.962) (width 0.25) (layer F.Cu) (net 19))
 (segment (start 136.906 76.962) (end 136.906 75.692) (width 0.25) (layer F.Cu) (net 19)))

